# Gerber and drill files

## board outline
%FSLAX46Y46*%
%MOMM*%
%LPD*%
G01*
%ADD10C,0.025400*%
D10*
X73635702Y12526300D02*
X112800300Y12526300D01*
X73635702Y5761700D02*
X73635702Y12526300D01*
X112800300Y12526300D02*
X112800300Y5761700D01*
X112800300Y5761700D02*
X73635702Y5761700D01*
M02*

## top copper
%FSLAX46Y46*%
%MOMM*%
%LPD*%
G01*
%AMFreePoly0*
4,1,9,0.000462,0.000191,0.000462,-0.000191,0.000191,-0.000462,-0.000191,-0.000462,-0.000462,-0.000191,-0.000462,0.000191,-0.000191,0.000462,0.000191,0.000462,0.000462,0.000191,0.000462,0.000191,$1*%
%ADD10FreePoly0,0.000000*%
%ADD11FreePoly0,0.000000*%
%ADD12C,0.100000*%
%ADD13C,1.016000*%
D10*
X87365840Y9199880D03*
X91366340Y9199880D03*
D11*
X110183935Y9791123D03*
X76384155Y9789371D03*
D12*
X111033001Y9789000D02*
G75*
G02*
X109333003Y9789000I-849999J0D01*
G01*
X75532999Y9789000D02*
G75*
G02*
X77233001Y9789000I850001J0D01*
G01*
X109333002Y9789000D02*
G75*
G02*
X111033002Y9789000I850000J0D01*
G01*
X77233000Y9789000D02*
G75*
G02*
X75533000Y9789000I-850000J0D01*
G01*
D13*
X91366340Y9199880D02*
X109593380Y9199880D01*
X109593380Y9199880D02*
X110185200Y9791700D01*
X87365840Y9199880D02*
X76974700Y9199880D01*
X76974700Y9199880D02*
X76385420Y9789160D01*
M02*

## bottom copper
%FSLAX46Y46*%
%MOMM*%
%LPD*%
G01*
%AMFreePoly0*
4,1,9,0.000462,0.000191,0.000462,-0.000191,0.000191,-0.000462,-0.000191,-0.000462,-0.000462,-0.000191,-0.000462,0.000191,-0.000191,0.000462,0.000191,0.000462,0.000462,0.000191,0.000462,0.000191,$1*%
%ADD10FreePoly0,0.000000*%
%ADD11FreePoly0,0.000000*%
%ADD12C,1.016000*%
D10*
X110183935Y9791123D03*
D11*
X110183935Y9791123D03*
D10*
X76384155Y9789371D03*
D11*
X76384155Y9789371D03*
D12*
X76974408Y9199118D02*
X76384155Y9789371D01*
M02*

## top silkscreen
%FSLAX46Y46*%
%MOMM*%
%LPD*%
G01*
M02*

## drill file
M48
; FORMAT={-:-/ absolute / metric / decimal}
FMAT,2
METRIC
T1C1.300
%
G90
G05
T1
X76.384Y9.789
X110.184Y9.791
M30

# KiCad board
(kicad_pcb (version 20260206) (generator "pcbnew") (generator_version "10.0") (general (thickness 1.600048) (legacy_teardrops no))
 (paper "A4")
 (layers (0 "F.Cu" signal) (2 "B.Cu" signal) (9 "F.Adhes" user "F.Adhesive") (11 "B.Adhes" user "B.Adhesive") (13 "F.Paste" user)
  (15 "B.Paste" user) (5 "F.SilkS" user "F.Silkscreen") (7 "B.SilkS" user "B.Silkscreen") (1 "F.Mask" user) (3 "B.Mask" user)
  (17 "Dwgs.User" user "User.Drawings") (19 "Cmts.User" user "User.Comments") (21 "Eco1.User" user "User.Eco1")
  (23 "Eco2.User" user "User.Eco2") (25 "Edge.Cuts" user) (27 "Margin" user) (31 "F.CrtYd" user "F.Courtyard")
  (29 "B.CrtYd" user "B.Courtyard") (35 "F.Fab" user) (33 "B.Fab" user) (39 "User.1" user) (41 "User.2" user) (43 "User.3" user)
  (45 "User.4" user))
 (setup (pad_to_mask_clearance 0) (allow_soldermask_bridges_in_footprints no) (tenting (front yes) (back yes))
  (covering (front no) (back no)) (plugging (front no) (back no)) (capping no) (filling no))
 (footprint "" (layer "F.Cu") (at 0 0)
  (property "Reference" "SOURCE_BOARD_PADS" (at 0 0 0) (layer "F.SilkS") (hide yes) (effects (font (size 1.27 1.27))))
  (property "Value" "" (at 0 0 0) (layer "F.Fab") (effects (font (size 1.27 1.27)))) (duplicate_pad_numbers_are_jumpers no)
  (pad "1" smd custom (at 87.36584 -9.19988) (size 0.001 0.001) (layers "F.Cu" "F.Mask" "F.Paste") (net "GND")
   (options (clearance outline) (anchor circle)) (primitives))
  (pad "2" smd custom (at 91.36634 -9.19988) (size 0.001 0.001) (layers "F.Cu" "F.Mask" "F.Paste") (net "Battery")
   (options (clearance outline) (anchor circle)) (primitives)))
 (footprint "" (layer "B.Cu") (at 110.183935 -9.791123)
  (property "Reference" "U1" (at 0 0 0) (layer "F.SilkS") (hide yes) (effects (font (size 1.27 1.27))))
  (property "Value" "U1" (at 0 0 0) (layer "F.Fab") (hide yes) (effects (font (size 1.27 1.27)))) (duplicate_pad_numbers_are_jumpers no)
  (pad "1" thru_hole custom (at 0 0) (size 0.001 0.001) (drill 1.300023) (layers "*.Cu") (remove_unused_layers no) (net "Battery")
   (options (clearance outline) (anchor circle)) (primitives))
  (pad "1" smd custom (at 0 0) (size 0.001 0.001) (layers "B.Cu" "B.Mask" "B.Paste") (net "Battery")
   (options (clearance outline) (anchor circle)) (primitives)))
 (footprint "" (layer "B.Cu") (at 76.384155 -9.789371)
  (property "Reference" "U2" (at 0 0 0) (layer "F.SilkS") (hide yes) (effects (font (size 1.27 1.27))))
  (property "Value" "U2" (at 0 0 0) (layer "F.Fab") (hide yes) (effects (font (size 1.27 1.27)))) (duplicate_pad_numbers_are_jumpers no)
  (pad "1" thru_hole custom (at 0 0) (size 0.001 0.001) (drill 1.300023) (layers "*.Cu") (remove_unused_layers no) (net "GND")
   (options (clearance outline) (anchor circle)) (primitives))
  (pad "1" smd custom (at 0 0) (size 0.001 0.001) (layers "B.Cu" "B.Mask" "B.Paste") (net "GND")
   (options (clearance outline) (anchor circle)) (primitives)))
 (gr_line (start 73.635702 -12.5263) (end 112.8003 -12.5263) (stroke (width 0.0254) (type default)) (layer "Edge.Cuts"))
 (gr_line (start 73.635702 -5.7617) (end 73.635702 -12.5263) (stroke (width 0.0254) (type default)) (layer "Edge.Cuts"))
 (gr_line (start 112.8003 -12.5263) (end 112.8003 -5.7617) (stroke (width 0.0254) (type default)) (layer "Edge.Cuts"))
 (gr_line (start 112.8003 -5.7617) (end 73.635702 -5.7617) (stroke (width 0.0254) (type default)) (layer "Edge.Cuts"))
 (arc (start 111.033001 -9.789) (mid 110.164713 -8.939197) (end 109.333002 -9.789) (width 0.1) (layer "F.Cu") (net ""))
 (arc (start 75.532999 -9.789) (mid 76.401288 -10.638804) (end 77.233 -9.789) (width 0.1) (layer "F.Cu") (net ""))
 (arc (start 109.333002 -9.789) (mid 110.20129 -10.638803) (end 111.033001 -9.789) (width 0.1) (layer "F.Cu") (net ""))
 (arc (start 77.233 -9.789) (mid 76.364711 -8.939196) (end 75.532999 -9.789) (width 0.1) (layer "F.Cu") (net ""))
 (segment (start 91.36634 -9.19988) (end 109.59338 -9.19988) (width 1.016) (layer "F.Cu") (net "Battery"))
 (segment (start 109.59338 -9.19988) (end 110.1852 -9.7917) (width 1.016) (layer "F.Cu") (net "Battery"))
 (segment (start 87.36584 -9.19988) (end 76.9747 -9.19988) (width 1.016) (layer "F.Cu") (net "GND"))
 (segment (start 76.9747 -9.19988) (end 76.38542 -9.78916) (width 1.016) (layer "F.Cu") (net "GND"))
 (segment (start 76.974408 -9.199118) (end 76.384155 -9.789371) (width 1.016) (layer "B.Cu") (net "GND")))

